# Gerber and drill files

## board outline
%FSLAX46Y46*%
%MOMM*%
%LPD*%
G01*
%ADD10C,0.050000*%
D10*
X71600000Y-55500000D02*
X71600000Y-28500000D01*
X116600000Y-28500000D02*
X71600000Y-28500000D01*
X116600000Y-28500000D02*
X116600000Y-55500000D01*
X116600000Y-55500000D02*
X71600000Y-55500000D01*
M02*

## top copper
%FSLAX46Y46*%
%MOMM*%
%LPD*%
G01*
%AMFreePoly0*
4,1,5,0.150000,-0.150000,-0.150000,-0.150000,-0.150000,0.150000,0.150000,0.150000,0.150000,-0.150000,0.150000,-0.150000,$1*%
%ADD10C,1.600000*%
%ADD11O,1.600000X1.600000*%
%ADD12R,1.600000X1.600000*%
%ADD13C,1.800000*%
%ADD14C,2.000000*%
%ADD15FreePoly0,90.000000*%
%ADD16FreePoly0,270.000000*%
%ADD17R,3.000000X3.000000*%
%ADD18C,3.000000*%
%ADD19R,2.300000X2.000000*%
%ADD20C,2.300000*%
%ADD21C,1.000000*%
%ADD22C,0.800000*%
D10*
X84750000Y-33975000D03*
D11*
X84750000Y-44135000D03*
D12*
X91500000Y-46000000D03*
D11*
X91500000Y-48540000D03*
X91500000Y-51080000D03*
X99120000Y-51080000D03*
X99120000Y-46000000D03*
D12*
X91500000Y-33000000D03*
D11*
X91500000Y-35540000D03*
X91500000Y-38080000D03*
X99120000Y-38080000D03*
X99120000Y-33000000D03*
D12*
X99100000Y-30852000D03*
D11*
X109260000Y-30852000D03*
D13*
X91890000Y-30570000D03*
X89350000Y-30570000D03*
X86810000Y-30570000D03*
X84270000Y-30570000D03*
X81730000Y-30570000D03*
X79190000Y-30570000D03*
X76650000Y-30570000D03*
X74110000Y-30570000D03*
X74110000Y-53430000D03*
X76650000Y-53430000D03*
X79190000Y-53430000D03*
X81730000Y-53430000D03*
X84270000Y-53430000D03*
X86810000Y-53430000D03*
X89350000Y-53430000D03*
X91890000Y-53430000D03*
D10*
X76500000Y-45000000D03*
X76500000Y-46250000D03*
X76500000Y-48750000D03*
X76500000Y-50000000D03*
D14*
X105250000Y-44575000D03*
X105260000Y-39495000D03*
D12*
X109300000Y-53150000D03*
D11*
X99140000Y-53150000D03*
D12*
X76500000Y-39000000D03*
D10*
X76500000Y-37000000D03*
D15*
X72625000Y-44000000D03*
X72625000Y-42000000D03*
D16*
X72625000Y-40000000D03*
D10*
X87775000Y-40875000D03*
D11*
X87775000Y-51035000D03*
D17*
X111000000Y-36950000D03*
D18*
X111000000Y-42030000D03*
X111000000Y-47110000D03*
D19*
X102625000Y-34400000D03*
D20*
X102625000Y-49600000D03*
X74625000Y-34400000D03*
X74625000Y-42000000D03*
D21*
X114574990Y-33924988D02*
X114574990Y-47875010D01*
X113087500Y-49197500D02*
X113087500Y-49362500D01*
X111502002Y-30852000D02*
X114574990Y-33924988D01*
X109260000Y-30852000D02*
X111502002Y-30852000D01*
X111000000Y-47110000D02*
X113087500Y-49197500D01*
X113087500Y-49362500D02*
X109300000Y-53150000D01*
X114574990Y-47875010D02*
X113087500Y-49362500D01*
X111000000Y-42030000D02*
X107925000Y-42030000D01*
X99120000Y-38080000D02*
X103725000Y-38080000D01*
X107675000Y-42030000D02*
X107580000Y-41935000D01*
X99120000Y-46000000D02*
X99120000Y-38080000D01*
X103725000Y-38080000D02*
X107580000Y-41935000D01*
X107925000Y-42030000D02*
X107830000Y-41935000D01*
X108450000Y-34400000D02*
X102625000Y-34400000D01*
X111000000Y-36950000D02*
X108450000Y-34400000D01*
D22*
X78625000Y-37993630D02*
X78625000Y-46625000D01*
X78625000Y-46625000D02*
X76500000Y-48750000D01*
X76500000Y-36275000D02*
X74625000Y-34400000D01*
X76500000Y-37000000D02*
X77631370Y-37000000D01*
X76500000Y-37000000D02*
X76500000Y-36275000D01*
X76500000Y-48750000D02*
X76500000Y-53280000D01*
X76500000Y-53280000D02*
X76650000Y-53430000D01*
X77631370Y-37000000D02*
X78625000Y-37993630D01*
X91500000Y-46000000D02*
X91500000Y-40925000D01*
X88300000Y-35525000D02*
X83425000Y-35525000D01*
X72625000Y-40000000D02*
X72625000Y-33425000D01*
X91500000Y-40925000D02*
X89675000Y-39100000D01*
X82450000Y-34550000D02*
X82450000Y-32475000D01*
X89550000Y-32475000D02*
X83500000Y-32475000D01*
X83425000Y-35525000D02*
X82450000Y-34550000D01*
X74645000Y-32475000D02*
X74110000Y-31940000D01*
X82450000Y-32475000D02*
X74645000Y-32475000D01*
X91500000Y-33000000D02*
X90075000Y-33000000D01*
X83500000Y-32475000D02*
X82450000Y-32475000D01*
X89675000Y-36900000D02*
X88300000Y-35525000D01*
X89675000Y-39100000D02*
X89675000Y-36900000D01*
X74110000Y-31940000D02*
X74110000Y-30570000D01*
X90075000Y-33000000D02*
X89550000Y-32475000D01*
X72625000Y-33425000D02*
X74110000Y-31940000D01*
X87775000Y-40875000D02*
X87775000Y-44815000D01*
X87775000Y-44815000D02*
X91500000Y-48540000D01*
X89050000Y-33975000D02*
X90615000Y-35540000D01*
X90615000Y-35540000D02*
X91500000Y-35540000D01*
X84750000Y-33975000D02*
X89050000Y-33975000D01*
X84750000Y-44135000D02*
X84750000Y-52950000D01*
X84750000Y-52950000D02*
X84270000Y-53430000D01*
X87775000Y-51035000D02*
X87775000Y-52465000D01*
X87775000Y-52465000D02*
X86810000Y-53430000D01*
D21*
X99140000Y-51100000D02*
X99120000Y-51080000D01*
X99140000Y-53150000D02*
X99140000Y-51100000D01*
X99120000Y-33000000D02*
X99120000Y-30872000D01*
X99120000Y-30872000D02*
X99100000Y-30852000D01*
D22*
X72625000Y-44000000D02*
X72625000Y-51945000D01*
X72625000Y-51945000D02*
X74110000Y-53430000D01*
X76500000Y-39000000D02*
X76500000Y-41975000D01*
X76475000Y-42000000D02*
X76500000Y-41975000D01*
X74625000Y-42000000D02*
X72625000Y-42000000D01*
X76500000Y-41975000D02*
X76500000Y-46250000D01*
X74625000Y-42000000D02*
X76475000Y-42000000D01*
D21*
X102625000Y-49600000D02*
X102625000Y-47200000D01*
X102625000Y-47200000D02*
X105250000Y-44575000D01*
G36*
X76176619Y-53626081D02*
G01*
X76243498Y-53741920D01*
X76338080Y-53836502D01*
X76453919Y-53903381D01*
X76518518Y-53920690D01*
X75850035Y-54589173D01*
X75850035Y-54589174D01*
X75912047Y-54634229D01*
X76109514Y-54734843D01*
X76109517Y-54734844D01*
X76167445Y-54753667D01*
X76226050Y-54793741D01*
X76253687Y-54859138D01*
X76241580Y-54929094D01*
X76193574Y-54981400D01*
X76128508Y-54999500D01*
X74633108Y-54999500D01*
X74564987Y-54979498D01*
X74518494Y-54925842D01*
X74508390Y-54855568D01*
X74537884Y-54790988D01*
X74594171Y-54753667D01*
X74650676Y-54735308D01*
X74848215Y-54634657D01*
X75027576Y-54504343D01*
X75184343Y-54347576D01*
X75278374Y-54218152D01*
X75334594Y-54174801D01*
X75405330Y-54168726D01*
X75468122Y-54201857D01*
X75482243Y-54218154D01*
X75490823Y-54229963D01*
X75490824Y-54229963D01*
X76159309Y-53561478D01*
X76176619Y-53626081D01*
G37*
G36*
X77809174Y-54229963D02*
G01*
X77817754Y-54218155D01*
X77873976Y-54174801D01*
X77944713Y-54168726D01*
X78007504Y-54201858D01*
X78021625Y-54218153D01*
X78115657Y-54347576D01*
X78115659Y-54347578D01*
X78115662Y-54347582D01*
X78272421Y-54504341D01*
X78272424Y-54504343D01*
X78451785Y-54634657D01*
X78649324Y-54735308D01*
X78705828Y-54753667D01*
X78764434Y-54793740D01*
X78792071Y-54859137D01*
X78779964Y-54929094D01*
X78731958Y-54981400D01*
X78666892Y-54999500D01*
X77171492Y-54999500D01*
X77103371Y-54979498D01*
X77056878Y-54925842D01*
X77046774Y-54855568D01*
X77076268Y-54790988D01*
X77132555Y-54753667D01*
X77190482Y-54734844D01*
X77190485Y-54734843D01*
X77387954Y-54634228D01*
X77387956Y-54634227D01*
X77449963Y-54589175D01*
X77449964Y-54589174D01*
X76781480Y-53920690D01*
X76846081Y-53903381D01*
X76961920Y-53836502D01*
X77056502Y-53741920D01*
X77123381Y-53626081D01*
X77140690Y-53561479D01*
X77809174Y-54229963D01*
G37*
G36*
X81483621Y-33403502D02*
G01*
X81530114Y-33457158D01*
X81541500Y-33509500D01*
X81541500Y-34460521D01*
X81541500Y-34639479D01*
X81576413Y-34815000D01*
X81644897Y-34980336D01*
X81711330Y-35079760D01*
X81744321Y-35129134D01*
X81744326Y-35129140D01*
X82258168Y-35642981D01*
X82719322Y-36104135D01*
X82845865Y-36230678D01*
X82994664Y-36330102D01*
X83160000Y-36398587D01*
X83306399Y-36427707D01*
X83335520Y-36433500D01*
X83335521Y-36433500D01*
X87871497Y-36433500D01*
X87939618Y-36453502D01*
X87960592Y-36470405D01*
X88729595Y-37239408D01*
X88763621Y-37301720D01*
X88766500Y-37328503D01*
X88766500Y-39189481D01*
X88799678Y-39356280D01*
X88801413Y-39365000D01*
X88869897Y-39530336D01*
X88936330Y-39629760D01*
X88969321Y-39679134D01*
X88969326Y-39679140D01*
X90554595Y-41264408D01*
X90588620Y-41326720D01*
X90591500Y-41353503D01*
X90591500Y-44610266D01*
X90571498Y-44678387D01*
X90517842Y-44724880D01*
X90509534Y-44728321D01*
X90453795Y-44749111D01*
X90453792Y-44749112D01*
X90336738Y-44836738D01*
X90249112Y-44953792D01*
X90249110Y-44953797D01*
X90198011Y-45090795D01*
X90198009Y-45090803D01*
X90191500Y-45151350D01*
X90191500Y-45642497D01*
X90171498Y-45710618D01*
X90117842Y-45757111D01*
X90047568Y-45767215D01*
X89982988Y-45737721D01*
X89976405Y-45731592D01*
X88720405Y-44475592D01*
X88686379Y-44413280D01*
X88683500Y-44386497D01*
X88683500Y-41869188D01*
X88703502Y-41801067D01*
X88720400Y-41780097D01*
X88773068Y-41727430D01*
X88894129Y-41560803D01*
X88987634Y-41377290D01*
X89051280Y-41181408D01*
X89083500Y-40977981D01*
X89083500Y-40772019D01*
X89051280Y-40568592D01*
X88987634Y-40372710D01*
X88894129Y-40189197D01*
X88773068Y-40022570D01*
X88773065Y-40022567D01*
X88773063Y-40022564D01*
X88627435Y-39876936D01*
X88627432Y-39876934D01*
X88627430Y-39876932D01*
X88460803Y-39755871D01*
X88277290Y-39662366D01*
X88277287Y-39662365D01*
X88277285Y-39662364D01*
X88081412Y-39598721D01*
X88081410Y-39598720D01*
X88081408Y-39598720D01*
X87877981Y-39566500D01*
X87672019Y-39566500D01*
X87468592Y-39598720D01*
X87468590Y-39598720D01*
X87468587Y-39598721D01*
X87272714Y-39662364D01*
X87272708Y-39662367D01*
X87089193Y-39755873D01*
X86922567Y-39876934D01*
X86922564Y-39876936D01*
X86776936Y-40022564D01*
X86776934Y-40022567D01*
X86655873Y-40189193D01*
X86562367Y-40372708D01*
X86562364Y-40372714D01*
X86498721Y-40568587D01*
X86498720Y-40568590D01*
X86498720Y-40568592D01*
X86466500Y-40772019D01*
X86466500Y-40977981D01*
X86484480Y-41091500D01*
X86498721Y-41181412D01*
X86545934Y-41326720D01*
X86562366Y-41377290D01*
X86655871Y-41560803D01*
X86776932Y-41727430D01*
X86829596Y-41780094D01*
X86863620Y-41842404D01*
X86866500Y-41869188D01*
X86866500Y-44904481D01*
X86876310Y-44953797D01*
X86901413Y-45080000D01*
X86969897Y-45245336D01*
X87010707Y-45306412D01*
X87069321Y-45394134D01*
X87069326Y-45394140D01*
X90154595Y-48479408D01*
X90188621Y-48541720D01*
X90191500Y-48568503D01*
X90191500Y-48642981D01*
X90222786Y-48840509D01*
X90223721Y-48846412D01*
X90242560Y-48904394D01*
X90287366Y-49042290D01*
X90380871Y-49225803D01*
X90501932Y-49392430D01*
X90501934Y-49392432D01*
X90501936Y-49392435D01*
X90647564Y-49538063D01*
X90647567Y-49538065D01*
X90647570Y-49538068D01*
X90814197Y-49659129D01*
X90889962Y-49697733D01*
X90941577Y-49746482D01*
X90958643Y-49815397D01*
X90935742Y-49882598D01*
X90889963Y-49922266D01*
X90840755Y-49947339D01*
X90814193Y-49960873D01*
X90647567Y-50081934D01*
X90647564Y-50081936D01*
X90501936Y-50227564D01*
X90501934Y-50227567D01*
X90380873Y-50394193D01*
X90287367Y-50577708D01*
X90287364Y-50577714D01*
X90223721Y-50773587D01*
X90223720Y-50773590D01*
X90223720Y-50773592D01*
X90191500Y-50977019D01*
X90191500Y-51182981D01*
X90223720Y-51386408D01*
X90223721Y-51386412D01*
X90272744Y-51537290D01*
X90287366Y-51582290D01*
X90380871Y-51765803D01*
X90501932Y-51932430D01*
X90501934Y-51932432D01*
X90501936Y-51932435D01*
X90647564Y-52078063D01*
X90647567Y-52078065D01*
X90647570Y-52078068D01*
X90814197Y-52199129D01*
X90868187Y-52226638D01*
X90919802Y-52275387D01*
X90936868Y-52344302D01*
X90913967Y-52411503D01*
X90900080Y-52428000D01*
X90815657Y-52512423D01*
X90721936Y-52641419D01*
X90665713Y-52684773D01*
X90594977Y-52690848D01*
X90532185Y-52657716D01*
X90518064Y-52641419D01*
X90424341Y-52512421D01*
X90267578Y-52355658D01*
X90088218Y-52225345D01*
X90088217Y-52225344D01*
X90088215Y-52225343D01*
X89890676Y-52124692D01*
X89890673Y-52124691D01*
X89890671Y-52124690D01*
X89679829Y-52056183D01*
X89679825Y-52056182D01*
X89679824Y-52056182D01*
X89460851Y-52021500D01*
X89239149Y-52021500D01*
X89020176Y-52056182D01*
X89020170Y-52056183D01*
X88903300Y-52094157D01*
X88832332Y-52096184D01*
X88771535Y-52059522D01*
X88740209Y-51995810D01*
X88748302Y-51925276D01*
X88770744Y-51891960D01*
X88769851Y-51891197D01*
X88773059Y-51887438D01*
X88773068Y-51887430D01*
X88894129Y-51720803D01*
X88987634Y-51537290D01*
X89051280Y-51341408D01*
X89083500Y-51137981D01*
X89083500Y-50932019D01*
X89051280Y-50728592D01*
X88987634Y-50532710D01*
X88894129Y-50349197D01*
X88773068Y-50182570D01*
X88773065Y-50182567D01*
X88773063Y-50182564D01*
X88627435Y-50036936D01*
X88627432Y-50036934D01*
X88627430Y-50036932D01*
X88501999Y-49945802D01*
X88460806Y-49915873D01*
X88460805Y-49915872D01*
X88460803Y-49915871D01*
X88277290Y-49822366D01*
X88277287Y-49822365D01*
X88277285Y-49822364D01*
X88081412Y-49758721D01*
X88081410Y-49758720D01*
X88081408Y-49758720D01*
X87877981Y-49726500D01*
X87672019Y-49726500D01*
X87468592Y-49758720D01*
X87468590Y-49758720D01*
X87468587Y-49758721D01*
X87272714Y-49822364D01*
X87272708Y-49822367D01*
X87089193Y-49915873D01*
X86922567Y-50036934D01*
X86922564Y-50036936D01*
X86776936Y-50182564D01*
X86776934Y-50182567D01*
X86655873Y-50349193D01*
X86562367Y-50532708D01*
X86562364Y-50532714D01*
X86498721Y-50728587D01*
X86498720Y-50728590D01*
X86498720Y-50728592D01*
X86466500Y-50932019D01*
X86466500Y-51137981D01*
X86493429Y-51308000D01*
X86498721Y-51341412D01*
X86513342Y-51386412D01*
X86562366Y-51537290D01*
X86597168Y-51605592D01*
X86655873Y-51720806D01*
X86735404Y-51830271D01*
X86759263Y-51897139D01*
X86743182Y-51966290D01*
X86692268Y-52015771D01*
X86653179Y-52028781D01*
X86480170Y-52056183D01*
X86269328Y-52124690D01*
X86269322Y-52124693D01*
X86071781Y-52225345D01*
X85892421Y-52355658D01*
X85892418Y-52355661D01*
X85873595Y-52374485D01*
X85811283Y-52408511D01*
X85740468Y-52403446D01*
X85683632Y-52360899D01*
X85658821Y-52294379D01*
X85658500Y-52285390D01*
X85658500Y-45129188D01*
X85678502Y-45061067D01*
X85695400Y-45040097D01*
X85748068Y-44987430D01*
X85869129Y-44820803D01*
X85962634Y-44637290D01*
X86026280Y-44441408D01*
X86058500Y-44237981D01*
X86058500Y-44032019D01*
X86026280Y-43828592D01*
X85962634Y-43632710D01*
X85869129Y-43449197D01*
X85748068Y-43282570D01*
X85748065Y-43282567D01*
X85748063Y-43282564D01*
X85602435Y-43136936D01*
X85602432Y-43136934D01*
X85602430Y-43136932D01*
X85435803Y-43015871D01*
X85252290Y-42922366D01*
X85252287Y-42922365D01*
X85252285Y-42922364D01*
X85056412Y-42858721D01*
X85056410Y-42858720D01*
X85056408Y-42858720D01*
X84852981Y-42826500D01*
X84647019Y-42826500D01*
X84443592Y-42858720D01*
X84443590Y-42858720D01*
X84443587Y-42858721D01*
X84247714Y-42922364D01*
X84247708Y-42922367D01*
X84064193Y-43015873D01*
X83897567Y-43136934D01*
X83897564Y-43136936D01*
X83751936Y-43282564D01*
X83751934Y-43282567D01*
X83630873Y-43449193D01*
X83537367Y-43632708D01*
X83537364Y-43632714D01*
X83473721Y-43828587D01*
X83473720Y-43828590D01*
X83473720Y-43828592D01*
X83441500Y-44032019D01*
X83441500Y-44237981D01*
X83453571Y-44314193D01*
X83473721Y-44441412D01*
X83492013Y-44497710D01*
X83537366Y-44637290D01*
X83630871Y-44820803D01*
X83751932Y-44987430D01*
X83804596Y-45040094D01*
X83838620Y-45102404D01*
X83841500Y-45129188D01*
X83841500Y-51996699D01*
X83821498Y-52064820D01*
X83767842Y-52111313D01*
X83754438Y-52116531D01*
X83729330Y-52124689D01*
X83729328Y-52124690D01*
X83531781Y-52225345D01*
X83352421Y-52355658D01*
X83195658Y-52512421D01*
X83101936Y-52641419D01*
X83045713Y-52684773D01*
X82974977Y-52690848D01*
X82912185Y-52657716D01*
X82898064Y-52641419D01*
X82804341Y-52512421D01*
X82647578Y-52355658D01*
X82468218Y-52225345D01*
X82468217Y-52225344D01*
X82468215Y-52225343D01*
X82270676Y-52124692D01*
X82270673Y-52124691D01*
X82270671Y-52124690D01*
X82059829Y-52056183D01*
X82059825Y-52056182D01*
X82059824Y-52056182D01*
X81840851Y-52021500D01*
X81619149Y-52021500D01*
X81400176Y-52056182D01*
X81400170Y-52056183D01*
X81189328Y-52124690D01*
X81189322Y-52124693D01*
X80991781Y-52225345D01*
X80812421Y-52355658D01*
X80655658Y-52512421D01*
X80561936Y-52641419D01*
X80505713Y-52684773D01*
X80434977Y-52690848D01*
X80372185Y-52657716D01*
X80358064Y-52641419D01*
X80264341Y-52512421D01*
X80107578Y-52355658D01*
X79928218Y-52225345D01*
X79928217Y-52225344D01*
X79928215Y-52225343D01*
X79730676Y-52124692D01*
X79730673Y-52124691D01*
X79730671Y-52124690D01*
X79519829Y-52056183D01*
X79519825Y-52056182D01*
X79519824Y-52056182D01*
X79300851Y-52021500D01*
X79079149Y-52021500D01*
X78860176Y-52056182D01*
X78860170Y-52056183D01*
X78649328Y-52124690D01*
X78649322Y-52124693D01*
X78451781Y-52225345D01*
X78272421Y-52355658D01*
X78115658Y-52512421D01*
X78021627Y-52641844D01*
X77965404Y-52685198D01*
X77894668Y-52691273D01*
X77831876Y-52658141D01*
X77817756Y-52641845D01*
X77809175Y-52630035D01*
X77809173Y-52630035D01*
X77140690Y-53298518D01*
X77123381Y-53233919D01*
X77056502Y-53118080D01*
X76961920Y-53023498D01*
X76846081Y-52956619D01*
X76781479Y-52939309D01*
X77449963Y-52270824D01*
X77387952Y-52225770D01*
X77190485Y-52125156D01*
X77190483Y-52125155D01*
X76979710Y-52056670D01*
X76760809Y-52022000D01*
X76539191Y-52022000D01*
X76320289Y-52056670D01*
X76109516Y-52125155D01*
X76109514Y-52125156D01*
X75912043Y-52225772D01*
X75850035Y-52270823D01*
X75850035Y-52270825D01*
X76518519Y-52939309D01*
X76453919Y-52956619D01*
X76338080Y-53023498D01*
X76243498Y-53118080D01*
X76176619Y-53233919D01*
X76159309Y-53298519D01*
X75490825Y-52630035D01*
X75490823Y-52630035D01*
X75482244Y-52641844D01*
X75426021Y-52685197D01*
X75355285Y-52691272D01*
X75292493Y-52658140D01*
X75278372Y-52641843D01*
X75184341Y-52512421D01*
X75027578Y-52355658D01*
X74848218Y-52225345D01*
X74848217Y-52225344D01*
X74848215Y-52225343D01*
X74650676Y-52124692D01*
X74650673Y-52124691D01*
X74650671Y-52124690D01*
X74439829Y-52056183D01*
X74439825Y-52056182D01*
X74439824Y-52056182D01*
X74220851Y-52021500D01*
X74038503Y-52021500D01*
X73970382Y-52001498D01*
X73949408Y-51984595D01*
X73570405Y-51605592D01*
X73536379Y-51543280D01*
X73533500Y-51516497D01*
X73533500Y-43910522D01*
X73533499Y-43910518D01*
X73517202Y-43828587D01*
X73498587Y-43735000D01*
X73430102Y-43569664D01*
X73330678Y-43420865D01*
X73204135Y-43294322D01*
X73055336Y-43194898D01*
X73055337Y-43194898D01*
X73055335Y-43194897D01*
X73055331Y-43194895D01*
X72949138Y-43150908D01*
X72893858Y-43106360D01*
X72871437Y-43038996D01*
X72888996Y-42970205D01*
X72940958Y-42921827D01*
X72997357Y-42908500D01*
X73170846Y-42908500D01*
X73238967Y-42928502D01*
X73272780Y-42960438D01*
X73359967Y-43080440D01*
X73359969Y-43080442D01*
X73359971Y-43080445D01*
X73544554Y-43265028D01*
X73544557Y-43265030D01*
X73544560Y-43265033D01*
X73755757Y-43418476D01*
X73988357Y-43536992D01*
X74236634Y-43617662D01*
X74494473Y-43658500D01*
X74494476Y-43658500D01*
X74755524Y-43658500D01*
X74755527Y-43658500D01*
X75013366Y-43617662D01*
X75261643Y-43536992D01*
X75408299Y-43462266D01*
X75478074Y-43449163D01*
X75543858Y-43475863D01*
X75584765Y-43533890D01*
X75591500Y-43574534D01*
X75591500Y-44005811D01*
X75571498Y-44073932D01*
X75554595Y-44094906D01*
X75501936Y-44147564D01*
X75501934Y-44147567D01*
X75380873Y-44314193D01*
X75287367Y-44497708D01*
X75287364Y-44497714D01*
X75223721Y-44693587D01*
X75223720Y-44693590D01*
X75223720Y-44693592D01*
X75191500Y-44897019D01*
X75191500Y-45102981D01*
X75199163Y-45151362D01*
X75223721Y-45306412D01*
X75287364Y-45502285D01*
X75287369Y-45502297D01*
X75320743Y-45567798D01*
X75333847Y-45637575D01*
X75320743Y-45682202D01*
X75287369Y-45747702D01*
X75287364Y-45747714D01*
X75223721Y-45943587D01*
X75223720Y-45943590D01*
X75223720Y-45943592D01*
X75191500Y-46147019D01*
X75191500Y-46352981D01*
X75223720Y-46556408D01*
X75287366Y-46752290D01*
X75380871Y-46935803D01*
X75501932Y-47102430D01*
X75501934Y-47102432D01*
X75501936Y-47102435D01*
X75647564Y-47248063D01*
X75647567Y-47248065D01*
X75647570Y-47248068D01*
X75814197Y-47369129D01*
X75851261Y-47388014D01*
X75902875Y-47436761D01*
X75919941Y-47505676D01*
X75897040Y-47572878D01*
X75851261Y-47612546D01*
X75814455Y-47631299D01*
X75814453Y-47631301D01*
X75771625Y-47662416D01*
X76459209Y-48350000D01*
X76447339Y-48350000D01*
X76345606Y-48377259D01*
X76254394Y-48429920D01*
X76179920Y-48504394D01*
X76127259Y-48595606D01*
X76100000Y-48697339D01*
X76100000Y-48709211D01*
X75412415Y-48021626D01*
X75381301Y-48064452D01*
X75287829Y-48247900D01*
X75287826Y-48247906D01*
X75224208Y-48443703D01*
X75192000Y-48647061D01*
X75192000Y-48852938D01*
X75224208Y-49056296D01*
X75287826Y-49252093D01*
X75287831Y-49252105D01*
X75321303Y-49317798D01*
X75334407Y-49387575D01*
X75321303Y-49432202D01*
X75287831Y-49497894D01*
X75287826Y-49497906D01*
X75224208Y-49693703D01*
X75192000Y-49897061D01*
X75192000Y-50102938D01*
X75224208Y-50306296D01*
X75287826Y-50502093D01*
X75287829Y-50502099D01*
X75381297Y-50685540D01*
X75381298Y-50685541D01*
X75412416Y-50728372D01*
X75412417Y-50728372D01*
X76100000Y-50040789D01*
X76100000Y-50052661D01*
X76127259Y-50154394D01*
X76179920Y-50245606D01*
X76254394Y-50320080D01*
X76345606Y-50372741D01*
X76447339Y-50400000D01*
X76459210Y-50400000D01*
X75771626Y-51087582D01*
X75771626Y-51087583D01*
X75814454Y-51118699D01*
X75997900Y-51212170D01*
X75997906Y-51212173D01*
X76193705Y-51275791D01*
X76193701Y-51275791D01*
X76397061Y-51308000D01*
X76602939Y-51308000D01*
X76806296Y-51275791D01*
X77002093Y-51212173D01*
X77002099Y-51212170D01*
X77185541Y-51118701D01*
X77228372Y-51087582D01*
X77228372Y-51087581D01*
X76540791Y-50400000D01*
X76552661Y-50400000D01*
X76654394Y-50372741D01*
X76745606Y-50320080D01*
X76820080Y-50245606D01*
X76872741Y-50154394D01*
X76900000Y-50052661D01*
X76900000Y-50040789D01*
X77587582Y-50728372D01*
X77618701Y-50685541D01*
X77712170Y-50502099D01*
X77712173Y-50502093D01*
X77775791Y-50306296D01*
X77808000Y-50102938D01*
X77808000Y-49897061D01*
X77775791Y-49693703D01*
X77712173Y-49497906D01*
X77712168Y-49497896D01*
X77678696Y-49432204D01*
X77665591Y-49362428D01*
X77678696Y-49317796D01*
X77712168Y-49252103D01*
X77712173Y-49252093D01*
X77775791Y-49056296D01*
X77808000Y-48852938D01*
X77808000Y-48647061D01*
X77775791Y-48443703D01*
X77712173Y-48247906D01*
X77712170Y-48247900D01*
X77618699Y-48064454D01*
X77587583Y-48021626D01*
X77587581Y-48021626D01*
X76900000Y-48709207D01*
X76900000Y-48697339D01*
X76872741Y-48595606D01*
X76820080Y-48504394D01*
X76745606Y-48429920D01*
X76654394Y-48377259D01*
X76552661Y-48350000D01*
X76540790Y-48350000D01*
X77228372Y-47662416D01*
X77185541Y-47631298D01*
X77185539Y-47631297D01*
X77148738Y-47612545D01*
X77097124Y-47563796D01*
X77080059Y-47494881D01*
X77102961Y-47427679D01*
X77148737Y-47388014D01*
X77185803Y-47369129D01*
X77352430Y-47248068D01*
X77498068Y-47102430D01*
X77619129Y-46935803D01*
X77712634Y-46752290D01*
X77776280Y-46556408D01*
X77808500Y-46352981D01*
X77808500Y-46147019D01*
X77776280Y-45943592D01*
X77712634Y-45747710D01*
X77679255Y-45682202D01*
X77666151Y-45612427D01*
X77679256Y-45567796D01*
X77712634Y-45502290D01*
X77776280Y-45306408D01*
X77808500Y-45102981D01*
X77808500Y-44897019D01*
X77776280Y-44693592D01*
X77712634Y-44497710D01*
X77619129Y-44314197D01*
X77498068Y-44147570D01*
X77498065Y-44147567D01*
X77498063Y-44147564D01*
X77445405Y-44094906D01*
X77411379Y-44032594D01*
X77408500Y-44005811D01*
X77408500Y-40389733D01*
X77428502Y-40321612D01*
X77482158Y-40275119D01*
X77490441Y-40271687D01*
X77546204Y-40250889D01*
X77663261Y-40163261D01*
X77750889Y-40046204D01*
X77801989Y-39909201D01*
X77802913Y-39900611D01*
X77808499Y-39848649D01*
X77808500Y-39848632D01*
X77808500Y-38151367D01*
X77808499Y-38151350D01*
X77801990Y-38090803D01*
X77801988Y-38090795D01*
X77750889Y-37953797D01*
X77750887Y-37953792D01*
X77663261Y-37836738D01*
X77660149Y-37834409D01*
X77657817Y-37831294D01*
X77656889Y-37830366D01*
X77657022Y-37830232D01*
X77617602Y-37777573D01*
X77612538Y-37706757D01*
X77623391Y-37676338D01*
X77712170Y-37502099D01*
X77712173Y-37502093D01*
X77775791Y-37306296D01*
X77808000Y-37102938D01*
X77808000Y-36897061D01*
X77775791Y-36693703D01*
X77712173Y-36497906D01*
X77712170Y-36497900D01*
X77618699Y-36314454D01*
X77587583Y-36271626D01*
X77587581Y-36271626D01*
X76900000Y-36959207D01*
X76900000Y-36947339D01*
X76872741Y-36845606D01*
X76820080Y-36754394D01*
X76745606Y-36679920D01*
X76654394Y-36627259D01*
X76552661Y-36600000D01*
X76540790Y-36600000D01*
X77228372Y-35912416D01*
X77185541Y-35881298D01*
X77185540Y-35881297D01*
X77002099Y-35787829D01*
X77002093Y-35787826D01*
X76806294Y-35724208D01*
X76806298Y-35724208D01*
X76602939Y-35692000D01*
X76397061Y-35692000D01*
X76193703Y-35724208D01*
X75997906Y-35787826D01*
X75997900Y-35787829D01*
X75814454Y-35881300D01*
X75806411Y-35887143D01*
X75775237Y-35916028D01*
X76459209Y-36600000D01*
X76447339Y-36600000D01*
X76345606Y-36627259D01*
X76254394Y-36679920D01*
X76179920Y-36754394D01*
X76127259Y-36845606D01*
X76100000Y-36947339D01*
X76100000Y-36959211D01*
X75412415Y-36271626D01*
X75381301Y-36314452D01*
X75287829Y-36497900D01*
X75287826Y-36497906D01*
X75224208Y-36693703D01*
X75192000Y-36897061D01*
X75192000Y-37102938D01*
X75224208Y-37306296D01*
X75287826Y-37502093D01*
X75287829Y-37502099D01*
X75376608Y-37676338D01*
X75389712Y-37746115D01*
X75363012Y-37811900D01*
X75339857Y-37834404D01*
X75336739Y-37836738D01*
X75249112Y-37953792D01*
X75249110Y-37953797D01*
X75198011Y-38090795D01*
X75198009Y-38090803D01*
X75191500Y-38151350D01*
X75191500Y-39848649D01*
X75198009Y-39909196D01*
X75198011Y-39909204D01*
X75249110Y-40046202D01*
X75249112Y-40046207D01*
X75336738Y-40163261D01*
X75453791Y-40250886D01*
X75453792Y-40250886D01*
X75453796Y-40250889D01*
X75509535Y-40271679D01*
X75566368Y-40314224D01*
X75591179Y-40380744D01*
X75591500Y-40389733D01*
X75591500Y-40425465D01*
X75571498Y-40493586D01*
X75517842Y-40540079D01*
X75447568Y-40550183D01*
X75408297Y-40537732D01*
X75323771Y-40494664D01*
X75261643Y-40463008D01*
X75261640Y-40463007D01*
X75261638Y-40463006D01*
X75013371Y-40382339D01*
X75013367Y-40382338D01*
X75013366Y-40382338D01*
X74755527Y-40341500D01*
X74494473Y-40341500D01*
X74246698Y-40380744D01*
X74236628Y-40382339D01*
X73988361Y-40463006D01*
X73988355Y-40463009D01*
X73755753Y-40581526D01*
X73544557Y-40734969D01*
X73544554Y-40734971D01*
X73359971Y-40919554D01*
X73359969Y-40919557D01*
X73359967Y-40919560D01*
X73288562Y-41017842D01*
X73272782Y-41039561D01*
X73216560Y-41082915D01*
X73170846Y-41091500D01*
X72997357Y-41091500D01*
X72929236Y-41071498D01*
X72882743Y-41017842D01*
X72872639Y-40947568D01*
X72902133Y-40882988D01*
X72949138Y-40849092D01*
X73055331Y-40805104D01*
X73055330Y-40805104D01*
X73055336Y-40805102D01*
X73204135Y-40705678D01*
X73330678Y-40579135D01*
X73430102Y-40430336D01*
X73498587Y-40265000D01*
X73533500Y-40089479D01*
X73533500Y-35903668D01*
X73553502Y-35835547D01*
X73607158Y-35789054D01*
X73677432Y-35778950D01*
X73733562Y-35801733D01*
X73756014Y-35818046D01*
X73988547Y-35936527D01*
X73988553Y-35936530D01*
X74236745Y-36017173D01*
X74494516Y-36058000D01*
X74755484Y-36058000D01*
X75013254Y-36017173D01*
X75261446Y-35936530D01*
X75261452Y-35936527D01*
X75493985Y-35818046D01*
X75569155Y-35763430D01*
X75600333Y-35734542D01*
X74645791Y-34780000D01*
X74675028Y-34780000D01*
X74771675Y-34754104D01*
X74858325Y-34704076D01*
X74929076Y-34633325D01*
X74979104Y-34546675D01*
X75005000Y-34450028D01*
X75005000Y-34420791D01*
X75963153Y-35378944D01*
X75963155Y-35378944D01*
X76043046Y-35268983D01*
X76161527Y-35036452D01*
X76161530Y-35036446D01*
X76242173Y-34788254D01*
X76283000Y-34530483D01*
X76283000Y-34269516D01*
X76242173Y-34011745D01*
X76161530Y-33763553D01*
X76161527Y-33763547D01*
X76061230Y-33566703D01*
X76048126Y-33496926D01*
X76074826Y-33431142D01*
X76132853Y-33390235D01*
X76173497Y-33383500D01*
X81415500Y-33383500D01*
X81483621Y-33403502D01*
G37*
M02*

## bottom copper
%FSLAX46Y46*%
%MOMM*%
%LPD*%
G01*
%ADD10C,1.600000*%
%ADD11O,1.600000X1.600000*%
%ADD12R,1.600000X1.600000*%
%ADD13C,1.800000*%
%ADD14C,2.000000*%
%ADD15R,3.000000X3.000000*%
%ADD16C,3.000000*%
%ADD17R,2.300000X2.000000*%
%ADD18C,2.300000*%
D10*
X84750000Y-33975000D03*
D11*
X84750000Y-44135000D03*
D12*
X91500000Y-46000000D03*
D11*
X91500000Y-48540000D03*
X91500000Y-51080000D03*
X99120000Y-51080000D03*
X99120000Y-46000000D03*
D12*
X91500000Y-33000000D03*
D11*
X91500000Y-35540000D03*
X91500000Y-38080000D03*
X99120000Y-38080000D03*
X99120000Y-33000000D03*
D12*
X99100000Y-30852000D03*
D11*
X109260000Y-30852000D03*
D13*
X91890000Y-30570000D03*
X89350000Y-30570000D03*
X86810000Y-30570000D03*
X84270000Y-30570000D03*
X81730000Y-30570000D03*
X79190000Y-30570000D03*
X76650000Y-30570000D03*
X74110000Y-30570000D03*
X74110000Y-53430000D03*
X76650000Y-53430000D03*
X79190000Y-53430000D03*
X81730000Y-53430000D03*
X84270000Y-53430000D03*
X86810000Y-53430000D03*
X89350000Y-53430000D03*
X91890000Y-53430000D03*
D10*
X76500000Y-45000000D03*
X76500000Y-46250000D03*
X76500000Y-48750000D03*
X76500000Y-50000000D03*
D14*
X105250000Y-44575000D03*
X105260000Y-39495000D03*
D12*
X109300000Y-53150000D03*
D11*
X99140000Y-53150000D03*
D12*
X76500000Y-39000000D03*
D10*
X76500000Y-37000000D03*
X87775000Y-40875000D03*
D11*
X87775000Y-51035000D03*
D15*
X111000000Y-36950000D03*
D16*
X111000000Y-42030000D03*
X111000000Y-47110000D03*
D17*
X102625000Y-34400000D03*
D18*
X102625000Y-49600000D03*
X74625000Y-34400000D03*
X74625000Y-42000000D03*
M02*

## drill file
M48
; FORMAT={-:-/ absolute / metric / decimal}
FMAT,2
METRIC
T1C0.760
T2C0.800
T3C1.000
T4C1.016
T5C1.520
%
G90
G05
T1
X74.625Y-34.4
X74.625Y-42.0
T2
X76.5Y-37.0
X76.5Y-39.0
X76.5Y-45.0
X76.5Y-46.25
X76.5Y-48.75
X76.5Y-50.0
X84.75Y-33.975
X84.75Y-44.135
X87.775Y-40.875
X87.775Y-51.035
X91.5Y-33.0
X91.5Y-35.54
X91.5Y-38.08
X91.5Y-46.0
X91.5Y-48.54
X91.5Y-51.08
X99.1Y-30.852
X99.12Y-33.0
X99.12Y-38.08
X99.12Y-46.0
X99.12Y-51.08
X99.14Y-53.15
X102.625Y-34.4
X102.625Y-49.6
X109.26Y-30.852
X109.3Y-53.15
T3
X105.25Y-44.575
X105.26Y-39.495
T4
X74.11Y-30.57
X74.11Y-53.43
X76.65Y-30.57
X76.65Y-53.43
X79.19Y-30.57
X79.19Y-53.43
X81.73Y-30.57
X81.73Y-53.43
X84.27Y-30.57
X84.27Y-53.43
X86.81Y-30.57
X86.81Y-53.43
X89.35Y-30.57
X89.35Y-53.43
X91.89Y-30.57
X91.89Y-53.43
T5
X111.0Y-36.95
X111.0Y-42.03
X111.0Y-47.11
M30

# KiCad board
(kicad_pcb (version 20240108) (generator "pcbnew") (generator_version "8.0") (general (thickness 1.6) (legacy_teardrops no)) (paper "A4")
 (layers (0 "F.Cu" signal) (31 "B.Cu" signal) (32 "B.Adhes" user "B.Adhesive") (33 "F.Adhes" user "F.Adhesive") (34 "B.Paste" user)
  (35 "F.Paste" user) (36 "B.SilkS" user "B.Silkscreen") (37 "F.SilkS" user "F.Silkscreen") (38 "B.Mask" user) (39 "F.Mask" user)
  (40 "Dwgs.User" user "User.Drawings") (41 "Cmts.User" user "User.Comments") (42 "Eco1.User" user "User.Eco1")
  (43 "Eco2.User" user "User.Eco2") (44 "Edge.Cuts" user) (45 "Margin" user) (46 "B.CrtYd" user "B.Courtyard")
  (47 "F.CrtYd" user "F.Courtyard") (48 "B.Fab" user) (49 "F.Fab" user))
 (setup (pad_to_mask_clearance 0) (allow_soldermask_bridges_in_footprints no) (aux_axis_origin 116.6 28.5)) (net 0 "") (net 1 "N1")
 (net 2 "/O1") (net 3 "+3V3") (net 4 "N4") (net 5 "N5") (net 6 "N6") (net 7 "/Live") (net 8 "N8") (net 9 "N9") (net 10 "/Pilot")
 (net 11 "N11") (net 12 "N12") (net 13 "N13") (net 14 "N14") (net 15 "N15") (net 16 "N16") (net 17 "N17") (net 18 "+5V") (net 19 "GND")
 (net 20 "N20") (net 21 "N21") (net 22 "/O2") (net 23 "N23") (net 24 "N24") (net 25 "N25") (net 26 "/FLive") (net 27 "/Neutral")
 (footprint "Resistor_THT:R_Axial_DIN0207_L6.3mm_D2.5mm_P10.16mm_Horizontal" (layer "F.Cu") (at 84.75 33.975 -90)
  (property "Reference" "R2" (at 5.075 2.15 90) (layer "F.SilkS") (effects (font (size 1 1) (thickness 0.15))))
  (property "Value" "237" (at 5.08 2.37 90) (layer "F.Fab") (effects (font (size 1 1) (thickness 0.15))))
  (pad "1" thru_hole circle (at 0 0 270) (size 1.6 1.6) (drill 0.8) (layers "*.Cu" "*.Mask") (remove_unused_layers no) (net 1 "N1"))
  (pad "2" thru_hole oval (at 10.16 0 270) (size 1.6 1.6) (drill 0.8) (layers "*.Cu" "*.Mask") (remove_unused_layers no) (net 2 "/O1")))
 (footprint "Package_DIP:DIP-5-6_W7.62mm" (layer "F.Cu") (at 91.5 46)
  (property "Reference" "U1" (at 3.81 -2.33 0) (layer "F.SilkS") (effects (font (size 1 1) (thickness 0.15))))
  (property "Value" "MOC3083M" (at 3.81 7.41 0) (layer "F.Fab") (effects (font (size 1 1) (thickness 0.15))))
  (pad "1" thru_hole rect (at 0 0) (size 1.6 1.6) (drill 0.8) (layers "*.Cu" "*.Mask") (remove_unused_layers no) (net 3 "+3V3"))
  (pad "2" thru_hole oval (at 0 2.54) (size 1.6 1.6) (drill 0.8) (layers "*.Cu" "*.Mask") (remove_unused_layers no) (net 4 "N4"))
  (pad "3" thru_hole oval (at 0 5.08) (size 1.6 1.6) (drill 0.8) (layers "*.Cu" "*.Mask") (remove_unused_layers no) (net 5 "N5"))
  (pad "4" thru_hole oval (at 7.62 5.08) (size 1.6 1.6) (drill 0.8) (layers "*.Cu" "*.Mask") (remove_unused_layers no) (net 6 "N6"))
  (pad "6" thru_hole oval (at 7.62 0) (size 1.6 1.6) (drill 0.8) (layers "*.Cu" "*.Mask") (remove_unused_layers no) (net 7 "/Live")))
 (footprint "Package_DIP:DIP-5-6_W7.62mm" (layer "F.Cu") (at 91.5 33)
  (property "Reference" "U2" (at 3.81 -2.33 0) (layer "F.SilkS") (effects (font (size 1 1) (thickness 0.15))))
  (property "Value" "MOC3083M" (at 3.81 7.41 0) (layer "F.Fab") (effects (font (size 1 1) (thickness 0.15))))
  (pad "1" thru_hole rect (at 0 0) (size 1.6 1.6) (drill 0.8) (layers "*.Cu" "*.Mask") (remove_unused_layers no) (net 3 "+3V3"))
  (pad "2" thru_hole oval (at 0 2.54) (size 1.6 1.6) (drill 0.8) (layers "*.Cu" "*.Mask") (remove_unused_layers no) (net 1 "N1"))
  (pad "3" thru_hole oval (at 0 5.08) (size 1.6 1.6) (drill 0.8) (layers "*.Cu" "*.Mask") (remove_unused_layers no) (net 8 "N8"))
  (pad "4" thru_hole oval (at 7.62 5.08) (size 1.6 1.6) (drill 0.8) (layers "*.Cu" "*.Mask") (remove_unused_layers no) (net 7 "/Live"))
  (pad "6" thru_hole oval (at 7.62 0) (size 1.6 1.6) (drill 0.8) (layers "*.Cu" "*.Mask") (remove_unused_layers no) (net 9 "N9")))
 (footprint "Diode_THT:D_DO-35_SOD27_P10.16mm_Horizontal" (layer "F.Cu") (at 99.1 30.852)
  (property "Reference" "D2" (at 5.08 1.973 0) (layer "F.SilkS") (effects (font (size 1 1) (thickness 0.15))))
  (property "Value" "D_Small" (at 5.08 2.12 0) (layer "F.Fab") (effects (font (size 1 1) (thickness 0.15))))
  (pad "1" thru_hole rect (at 0 0) (size 1.6 1.6) (drill 0.8) (layers "*.Cu" "*.Mask") (remove_unused_layers no) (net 9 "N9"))
  (pad "2" thru_hole oval (at 10.16 0) (size 1.6 1.6) (drill 0.8) (layers "*.Cu" "*.Mask") (remove_unused_layers no) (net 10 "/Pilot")))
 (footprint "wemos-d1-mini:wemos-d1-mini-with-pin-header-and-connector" (layer "F.Cu") (at 83 42)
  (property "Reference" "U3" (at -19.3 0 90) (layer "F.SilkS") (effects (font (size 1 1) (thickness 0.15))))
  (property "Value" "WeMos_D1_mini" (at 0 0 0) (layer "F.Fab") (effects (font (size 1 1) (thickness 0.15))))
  (pad "1" thru_hole circle (at 8.89 -11.43) (size 1.8 1.8) (drill 1.016) (layers "*.Cu" "*.Mask") (remove_unused_layers no) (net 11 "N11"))
  (pad "2" thru_hole circle (at 6.35 -11.43) (size 1.8 1.8) (drill 1.016) (layers "*.Cu" "*.Mask") (remove_unused_layers no) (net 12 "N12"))
  (pad "3" thru_hole circle (at 3.81 -11.43) (size 1.8 1.8) (drill 1.016) (layers "*.Cu" "*.Mask") (remove_unused_layers no) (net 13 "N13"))
  (pad "4" thru_hole circle (at 1.27 -11.43) (size 1.8 1.8) (drill 1.016) (layers "*.Cu" "*.Mask") (remove_unused_layers no) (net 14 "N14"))
  (pad "5" thru_hole circle (at -1.27 -11.43) (size 1.8 1.8) (drill 1.016) (layers "*.Cu" "*.Mask") (remove_unused_layers no) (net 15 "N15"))
  (pad "6" thru_hole circle (at -3.81 -11.43 90) (size 1.8 1.8) (drill 1.016) (layers "*.Cu" "*.Mask") (remove_unused_layers no)
   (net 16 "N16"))
  (pad "7" thru_hole circle (at -6.35 -11.43) (size 1.8 1.8) (drill 1.016) (layers "*.Cu" "*.Mask") (remove_unused_layers no) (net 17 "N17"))
  (pad "8" thru_hole circle (at -8.89 -11.43) (size 1.8 1.8) (drill 1.016) (layers "*.Cu" "*.Mask") (remove_unused_layers no) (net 3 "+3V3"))
  (pad "9" thru_hole circle (at -8.89 11.43) (size 1.8 1.8) (drill 1.016) (layers "*.Cu" "*.Mask") (remove_unused_layers no) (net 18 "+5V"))
  (pad "10" thru_hole circle (at -6.35 11.43) (size 1.8 1.8) (drill 1.016) (layers "*.Cu" "*.Mask") (remove_unused_layers no) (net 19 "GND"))
  (pad "11" thru_hole circle (at -3.81 11.43) (size 1.8 1.8) (drill 1.016) (layers "*.Cu" "*.Mask") (remove_unused_layers no) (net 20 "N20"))
  (pad "12" thru_hole circle (at -1.27 11.43) (size 1.8 1.8) (drill 1.016) (layers "*.Cu" "*.Mask") (remove_unused_layers no) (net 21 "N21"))
  (pad "13" thru_hole circle (at 1.27 11.43) (size 1.8 1.8) (drill 1.016) (layers "*.Cu" "*.Mask") (remove_unused_layers no) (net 2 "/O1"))
  (pad "14" thru_hole circle (at 3.81 11.43) (size 1.8 1.8) (drill 1.016) (layers "*.Cu" "*.Mask") (remove_unused_layers no) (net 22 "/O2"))
  (pad "15" thru_hole circle (at 6.35 11.43) (size 1.8 1.8) (drill 1.016) (layers "*.Cu" "*.Mask") (remove_unused_layers no) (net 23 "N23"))
  (pad "16" thru_hole circle (at 8.89 11.43) (size 1.8 1.8) (drill 1.016) (layers "*.Cu" "*.Mask") (remove_unused_layers no) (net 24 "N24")))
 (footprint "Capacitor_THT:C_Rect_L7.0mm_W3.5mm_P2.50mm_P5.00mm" (layer "F.Cu") (at 76.5 45 -90)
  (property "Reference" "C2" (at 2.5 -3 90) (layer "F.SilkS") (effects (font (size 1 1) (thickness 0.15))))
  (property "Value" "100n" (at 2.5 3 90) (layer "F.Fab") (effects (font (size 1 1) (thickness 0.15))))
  (pad "1" thru_hole circle (at 0 0 270) (size 1.6 1.6) (drill 0.8) (layers "*.Cu" "*.Mask") (remove_unused_layers no) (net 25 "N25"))
  (pad "1" thru_hole circle (at 1.25 0 270) (size 1.6 1.6) (drill 0.8) (layers "*.Cu" "*.Mask") (remove_unused_layers no) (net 25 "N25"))
  (pad "2" thru_hole circle (at 3.75 0 270) (size 1.6 1.6) (drill 0.8) (layers "*.Cu" "*.Mask") (remove_unused_layers no) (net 19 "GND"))
  (pad "2" thru_hole circle (at 5 0 270) (size 1.6 1.6) (drill 0.8) (layers "*.Cu" "*.Mask") (remove_unused_layers no) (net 19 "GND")))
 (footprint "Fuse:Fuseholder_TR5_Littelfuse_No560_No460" (layer "F.Cu") (at 105.25 44.575 90)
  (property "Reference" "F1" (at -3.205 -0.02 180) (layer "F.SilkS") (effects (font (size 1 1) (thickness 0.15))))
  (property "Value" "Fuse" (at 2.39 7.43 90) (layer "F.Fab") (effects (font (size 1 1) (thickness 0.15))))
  (pad "1" thru_hole circle (at 0 0 90) (size 2 2) (drill 1) (layers "*.Cu" "*.Mask") (remove_unused_layers no) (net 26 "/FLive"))
  (pad "2" thru_hole circle (at 5.08 0.01 90) (size 2 2) (drill 1) (layers "*.Cu" "*.Mask") (remove_unused_layers no) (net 7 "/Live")))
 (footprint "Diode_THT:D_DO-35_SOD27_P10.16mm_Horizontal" (layer "F.Cu") (at 109.3 53.15 180)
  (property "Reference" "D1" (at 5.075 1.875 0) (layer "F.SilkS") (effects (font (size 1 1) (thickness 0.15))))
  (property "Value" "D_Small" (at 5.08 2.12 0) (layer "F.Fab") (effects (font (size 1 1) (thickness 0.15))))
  (pad "1" thru_hole rect (at 0 0 180) (size 1.6 1.6) (drill 0.8) (layers "*.Cu" "*.Mask") (remove_unused_layers no) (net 10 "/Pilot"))
  (pad "2" thru_hole oval (at 10.16 0 180) (size 1.6 1.6) (drill 0.8) (layers "*.Cu" "*.Mask") (remove_unused_layers no) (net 6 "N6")))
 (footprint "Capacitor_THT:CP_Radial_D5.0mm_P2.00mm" (layer "F.Cu") (at 76.5 39 90)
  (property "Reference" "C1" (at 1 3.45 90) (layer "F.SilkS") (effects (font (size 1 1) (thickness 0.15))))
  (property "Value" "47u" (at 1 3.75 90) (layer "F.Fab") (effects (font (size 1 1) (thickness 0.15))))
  (pad "1" thru_hole rect (at 0 0 90) (size 1.6 1.6) (drill 0.8) (layers "*.Cu" "*.Mask") (remove_unused_layers no) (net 25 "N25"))
  (pad "2" thru_hole circle (at 2 0 90) (size 1.6 1.6) (drill 0.8) (layers "*.Cu" "*.Mask") (remove_unused_layers no) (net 19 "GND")))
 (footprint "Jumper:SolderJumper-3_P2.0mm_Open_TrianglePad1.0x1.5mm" (layer "F.Cu") (at 72.625 42 90)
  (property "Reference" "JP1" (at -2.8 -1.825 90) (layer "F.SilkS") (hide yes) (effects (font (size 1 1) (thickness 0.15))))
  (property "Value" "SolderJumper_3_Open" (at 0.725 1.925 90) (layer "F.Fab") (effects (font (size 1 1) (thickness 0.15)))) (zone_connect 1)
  (pad "" smd rect (at -1.2 0 90) (size 1.5 1.5) (layers "F.Mask"))
  (pad "" smd rect (at 1.2 0 90) (size 1.5 1.5) (layers "F.Mask"))
  (pad "1" smd custom (at -2 0 90) (size 0.3 0.3) (layers "F.Cu" "F.Mask") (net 18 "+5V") (zone_connect 2) (thermal_bridge_angle 45)
   (options (clearance outline) (anchor rect)) (primitives))
  (pad "2" smd custom (at 0 0 90) (size 0.3 0.3) (layers "F.Cu") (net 25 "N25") (zone_connect 2) (thermal_bridge_angle 45)
   (options (clearance outline) (anchor rect)) (primitives))
  (pad "3" smd custom (at 2 0 270) (size 0.3 0.3) (layers "F.Cu" "F.Mask") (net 3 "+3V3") (zone_connect 2) (thermal_bridge_angle 45)
   (options (clearance outline) (anchor rect)) (primitives)))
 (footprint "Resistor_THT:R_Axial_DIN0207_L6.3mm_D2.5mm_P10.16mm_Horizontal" (layer "F.Cu") (at 87.775 40.875 -90)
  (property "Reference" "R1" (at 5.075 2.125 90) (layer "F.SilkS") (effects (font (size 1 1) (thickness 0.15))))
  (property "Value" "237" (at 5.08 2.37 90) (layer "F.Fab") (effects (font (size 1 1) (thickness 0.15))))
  (pad "1" thru_hole circle (at 0 0 270) (size 1.6 1.6) (drill 0.8) (layers "*.Cu" "*.Mask") (remove_unused_layers no) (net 4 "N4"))
  (pad "2" thru_hole oval (at 10.16 0 270) (size 1.6 1.6) (drill 0.8) (layers "*.Cu" "*.Mask") (remove_unused_layers no) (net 22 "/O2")))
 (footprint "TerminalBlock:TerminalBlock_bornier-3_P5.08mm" (layer "B.Cu") (at 111 36.95 -90)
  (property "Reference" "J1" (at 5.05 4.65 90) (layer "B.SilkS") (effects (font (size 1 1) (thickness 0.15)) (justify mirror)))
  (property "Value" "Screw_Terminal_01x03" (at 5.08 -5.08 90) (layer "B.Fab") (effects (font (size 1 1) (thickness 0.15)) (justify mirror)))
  (pad "1" thru_hole rect (at 0 0 270) (size 3 3) (drill 1.52) (layers "*.Cu" "*.Mask") (remove_unused_layers no) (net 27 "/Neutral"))
  (pad "2" thru_hole circle (at 5.08 0 270) (size 3 3) (drill 1.52) (layers "*.Cu" "*.Mask") (remove_unused_layers no) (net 7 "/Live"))
  (pad "3" thru_hole circle (at 10.16 0 270) (size 3 3) (drill 1.52) (layers "*.Cu" "*.Mask") (remove_unused_layers no) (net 10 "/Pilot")))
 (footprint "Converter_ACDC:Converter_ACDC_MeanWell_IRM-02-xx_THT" (layer "B.Cu") (at 102.625 34.4 180)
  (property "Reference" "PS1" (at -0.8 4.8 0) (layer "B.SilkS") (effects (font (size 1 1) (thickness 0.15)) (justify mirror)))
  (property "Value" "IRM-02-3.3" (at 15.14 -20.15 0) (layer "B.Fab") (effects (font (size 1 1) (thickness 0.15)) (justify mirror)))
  (pad "1" thru_hole rect (at 0 0 180) (size 2.3 2) (drill 0.8) (layers "*.Cu" "*.Mask") (remove_unused_layers no) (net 27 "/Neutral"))
  (pad "2" thru_hole circle (at 0 -15.2 180) (size 2.3 2.3) (drill 0.8) (layers "*.Cu" "*.Mask") (remove_unused_layers no) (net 26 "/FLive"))
  (pad "3" thru_hole circle (at 28 0 180) (size 2.3 2.3) (drill 0.76) (layers "*.Cu" "*.Mask") (remove_unused_layers no) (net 19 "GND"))
  (pad "4" thru_hole circle (at 28 -7.6 180) (size 2.3 2.3) (drill 0.76) (layers "*.Cu" "*.Mask") (remove_unused_layers no) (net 25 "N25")))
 (gr_line (start 71.6 55.5) (end 71.6 28.5) (stroke (width 0.05) (type solid)) (layer "Edge.Cuts"))
 (gr_line (start 116.6 28.5) (end 71.6 28.5) (stroke (width 0.05) (type solid)) (layer "Edge.Cuts"))
 (gr_line (start 116.6 28.5) (end 116.6 55.5) (stroke (width 0.05) (type solid)) (layer "Edge.Cuts"))
 (gr_line (start 116.6 55.5) (end 71.6 55.5) (stroke (width 0.05) (type solid)) (layer "Edge.Cuts"))
 (segment (start 114.57499 33.924988) (end 114.57499 47.87501) (width 1) (layer "F.Cu") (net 10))
 (segment (start 113.0875 49.1975) (end 113.0875 49.3625) (width 1) (layer "F.Cu") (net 10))
 (segment (start 111.502002 30.852) (end 114.57499 33.924988) (width 1) (layer "F.Cu") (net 10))
 (segment (start 109.26 30.852) (end 111.502002 30.852) (width 1) (layer "F.Cu") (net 10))
 (segment (start 111 47.11) (end 113.0875 49.1975) (width 1) (layer "F.Cu") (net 10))
 (segment (start 113.0875 49.3625) (end 109.3 53.15) (width 1) (layer "F.Cu") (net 10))
 (segment (start 114.57499 47.87501) (end 113.0875 49.3625) (width 1) (layer "F.Cu") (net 10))
 (segment (start 111 42.03) (end 107.925 42.03) (width 1) (layer "F.Cu") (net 7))
 (segment (start 99.12 38.08) (end 103.725 38.08) (width 1) (layer "F.Cu") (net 7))
 (segment (start 107.675 42.03) (end 107.58 41.935) (width 1) (layer "F.Cu") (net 7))
 (segment (start 99.12 46) (end 99.12 38.08) (width 1) (layer "F.Cu") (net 7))
 (segment (start 103.725 38.08) (end 107.58 41.935) (width 1) (layer "F.Cu") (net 7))
 (segment (start 107.925 42.03) (end 107.83 41.935) (width 1) (layer "F.Cu") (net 7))
 (segment (start 108.45 34.4) (end 102.625 34.4) (width 1) (layer "F.Cu") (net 27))
 (segment (start 111 36.95) (end 108.45 34.4) (width 1) (layer "F.Cu") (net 27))
 (segment (start 78.625 37.99363) (end 78.625 46.625) (width 0.8) (layer "F.Cu") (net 19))
 (segment (start 78.625 46.625) (end 76.5 48.75) (width 0.8) (layer "F.Cu") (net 19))
 (segment (start 76.5 36.275) (end 74.625 34.4) (width 0.8) (layer "F.Cu") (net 19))
 (segment (start 76.5 37) (end 77.63137 37) (width 0.8) (layer "F.Cu") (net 19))
 (segment (start 76.5 37) (end 76.5 36.275) (width 0.8) (layer "F.Cu") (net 19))
 (segment (start 76.5 48.75) (end 76.5 53.28) (width 0.8) (layer "F.Cu") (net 19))
 (segment (start 76.5 53.28) (end 76.65 53.43) (width 0.8) (layer "F.Cu") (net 19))
 (segment (start 77.63137 37) (end 78.625 37.99363) (width 0.8) (layer "F.Cu") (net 19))
 (segment (start 91.5 46) (end 91.5 40.925) (width 0.8) (layer "F.Cu") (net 3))
 (segment (start 88.3 35.525) (end 83.425 35.525) (width 0.8) (layer "F.Cu") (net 3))
 (segment (start 72.625 40) (end 72.625 33.425) (width 0.8) (layer "F.Cu") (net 3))
 (segment (start 91.5 40.925) (end 89.675 39.1) (width 0.8) (layer "F.Cu") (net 3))
 (segment (start 82.45 34.55) (end 82.45 32.475) (width 0.8) (layer "F.Cu") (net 3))
 (segment (start 89.55 32.475) (end 83.5 32.475) (width 0.8) (layer "F.Cu") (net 3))
 (segment (start 83.425 35.525) (end 82.45 34.55) (width 0.8) (layer "F.Cu") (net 3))
 (segment (start 74.645 32.475) (end 74.11 31.94) (width 0.8) (layer "F.Cu") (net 3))
 (segment (start 82.45 32.475) (end 74.645 32.475) (width 0.8) (layer "F.Cu") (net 3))
 (segment (start 91.5 33) (end 90.075 33) (width 0.8) (layer "F.Cu") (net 3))
 (segment (start 83.5 32.475) (end 82.45 32.475) (width 0.8) (layer "F.Cu") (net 3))
 (segment (start 89.675 36.9) (end 88.3 35.525) (width 0.8) (layer "F.Cu") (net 3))
 (segment (start 89.675 39.1) (end 89.675 36.9) (width 0.8) (layer "F.Cu") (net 3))
 (segment (start 74.11 31.94) (end 74.11 30.57) (width 0.8) (layer "F.Cu") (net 3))
 (segment (start 90.075 33) (end 89.55 32.475) (width 0.8) (layer "F.Cu") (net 3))
 (segment (start 72.625 33.425) (end 74.11 31.94) (width 0.8) (layer "F.Cu") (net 3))
 (segment (start 87.775 40.875) (end 87.775 44.815) (width 0.8) (layer "F.Cu") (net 4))
 (segment (start 87.775 44.815) (end 91.5 48.54) (width 0.8) (layer "F.Cu") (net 4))
 (segment (start 89.05 33.975) (end 90.615 35.54) (width 0.8) (layer "F.Cu") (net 1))
 (segment (start 90.615 35.54) (end 91.5 35.54) (width 0.8) (layer "F.Cu") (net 1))
 (segment (start 84.75 33.975) (end 89.05 33.975) (width 0.8) (layer "F.Cu") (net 1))
 (segment (start 84.75 44.135) (end 84.75 52.95) (width 0.8) (layer "F.Cu") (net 2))
 (segment (start 84.75 52.95) (end 84.27 53.43) (width 0.8) (layer "F.Cu") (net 2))
 (segment (start 87.775 51.035) (end 87.775 52.465) (width 0.8) (layer "F.Cu") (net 22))
 (segment (start 87.775 52.465) (end 86.81 53.43) (width 0.8) (layer "F.Cu") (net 22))
 (segment (start 99.14 51.1) (end 99.12 51.08) (width 1) (layer "F.Cu") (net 6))
 (segment (start 99.14 53.15) (end 99.14 51.1) (width 1) (layer "F.Cu") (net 6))
 (segment (start 99.12 33) (end 99.12 30.872) (width 1) (layer "F.Cu") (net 9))
 (segment (start 99.12 30.872) (end 99.1 30.852) (width 1) (layer "F.Cu") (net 9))
 (segment (start 72.625 44) (end 72.625 51.945) (width 0.8) (layer "F.Cu") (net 18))
 (segment (start 72.625 51.945) (end 74.11 53.43) (width 0.8) (layer "F.Cu") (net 18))
 (segment (start 76.5 39) (end 76.5 41.975) (width 0.8) (layer "F.Cu") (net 25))
 (segment (start 76.475 42) (end 76.5 41.975) (width 0.8) (layer "F.Cu") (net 25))
 (segment (start 74.625 42) (end 72.625 42) (width 0.8) (layer "F.Cu") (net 25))
 (segment (start 76.5 41.975) (end 76.5 46.25) (width 0.8) (layer "F.Cu") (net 25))
 (segment (start 74.625 42) (end 76.475 42) (width 0.8) (layer "F.Cu") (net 25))
 (segment (start 102.625 49.6) (end 102.625 47.2) (width 1) (layer "F.Cu") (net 26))
 (segment (start 102.625 47.2) (end 105.25 44.575) (width 1) (layer "F.Cu") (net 26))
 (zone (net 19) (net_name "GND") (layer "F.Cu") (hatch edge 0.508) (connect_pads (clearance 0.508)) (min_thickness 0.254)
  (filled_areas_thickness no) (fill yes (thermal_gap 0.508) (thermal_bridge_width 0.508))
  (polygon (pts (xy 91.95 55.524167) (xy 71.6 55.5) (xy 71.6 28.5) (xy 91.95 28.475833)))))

